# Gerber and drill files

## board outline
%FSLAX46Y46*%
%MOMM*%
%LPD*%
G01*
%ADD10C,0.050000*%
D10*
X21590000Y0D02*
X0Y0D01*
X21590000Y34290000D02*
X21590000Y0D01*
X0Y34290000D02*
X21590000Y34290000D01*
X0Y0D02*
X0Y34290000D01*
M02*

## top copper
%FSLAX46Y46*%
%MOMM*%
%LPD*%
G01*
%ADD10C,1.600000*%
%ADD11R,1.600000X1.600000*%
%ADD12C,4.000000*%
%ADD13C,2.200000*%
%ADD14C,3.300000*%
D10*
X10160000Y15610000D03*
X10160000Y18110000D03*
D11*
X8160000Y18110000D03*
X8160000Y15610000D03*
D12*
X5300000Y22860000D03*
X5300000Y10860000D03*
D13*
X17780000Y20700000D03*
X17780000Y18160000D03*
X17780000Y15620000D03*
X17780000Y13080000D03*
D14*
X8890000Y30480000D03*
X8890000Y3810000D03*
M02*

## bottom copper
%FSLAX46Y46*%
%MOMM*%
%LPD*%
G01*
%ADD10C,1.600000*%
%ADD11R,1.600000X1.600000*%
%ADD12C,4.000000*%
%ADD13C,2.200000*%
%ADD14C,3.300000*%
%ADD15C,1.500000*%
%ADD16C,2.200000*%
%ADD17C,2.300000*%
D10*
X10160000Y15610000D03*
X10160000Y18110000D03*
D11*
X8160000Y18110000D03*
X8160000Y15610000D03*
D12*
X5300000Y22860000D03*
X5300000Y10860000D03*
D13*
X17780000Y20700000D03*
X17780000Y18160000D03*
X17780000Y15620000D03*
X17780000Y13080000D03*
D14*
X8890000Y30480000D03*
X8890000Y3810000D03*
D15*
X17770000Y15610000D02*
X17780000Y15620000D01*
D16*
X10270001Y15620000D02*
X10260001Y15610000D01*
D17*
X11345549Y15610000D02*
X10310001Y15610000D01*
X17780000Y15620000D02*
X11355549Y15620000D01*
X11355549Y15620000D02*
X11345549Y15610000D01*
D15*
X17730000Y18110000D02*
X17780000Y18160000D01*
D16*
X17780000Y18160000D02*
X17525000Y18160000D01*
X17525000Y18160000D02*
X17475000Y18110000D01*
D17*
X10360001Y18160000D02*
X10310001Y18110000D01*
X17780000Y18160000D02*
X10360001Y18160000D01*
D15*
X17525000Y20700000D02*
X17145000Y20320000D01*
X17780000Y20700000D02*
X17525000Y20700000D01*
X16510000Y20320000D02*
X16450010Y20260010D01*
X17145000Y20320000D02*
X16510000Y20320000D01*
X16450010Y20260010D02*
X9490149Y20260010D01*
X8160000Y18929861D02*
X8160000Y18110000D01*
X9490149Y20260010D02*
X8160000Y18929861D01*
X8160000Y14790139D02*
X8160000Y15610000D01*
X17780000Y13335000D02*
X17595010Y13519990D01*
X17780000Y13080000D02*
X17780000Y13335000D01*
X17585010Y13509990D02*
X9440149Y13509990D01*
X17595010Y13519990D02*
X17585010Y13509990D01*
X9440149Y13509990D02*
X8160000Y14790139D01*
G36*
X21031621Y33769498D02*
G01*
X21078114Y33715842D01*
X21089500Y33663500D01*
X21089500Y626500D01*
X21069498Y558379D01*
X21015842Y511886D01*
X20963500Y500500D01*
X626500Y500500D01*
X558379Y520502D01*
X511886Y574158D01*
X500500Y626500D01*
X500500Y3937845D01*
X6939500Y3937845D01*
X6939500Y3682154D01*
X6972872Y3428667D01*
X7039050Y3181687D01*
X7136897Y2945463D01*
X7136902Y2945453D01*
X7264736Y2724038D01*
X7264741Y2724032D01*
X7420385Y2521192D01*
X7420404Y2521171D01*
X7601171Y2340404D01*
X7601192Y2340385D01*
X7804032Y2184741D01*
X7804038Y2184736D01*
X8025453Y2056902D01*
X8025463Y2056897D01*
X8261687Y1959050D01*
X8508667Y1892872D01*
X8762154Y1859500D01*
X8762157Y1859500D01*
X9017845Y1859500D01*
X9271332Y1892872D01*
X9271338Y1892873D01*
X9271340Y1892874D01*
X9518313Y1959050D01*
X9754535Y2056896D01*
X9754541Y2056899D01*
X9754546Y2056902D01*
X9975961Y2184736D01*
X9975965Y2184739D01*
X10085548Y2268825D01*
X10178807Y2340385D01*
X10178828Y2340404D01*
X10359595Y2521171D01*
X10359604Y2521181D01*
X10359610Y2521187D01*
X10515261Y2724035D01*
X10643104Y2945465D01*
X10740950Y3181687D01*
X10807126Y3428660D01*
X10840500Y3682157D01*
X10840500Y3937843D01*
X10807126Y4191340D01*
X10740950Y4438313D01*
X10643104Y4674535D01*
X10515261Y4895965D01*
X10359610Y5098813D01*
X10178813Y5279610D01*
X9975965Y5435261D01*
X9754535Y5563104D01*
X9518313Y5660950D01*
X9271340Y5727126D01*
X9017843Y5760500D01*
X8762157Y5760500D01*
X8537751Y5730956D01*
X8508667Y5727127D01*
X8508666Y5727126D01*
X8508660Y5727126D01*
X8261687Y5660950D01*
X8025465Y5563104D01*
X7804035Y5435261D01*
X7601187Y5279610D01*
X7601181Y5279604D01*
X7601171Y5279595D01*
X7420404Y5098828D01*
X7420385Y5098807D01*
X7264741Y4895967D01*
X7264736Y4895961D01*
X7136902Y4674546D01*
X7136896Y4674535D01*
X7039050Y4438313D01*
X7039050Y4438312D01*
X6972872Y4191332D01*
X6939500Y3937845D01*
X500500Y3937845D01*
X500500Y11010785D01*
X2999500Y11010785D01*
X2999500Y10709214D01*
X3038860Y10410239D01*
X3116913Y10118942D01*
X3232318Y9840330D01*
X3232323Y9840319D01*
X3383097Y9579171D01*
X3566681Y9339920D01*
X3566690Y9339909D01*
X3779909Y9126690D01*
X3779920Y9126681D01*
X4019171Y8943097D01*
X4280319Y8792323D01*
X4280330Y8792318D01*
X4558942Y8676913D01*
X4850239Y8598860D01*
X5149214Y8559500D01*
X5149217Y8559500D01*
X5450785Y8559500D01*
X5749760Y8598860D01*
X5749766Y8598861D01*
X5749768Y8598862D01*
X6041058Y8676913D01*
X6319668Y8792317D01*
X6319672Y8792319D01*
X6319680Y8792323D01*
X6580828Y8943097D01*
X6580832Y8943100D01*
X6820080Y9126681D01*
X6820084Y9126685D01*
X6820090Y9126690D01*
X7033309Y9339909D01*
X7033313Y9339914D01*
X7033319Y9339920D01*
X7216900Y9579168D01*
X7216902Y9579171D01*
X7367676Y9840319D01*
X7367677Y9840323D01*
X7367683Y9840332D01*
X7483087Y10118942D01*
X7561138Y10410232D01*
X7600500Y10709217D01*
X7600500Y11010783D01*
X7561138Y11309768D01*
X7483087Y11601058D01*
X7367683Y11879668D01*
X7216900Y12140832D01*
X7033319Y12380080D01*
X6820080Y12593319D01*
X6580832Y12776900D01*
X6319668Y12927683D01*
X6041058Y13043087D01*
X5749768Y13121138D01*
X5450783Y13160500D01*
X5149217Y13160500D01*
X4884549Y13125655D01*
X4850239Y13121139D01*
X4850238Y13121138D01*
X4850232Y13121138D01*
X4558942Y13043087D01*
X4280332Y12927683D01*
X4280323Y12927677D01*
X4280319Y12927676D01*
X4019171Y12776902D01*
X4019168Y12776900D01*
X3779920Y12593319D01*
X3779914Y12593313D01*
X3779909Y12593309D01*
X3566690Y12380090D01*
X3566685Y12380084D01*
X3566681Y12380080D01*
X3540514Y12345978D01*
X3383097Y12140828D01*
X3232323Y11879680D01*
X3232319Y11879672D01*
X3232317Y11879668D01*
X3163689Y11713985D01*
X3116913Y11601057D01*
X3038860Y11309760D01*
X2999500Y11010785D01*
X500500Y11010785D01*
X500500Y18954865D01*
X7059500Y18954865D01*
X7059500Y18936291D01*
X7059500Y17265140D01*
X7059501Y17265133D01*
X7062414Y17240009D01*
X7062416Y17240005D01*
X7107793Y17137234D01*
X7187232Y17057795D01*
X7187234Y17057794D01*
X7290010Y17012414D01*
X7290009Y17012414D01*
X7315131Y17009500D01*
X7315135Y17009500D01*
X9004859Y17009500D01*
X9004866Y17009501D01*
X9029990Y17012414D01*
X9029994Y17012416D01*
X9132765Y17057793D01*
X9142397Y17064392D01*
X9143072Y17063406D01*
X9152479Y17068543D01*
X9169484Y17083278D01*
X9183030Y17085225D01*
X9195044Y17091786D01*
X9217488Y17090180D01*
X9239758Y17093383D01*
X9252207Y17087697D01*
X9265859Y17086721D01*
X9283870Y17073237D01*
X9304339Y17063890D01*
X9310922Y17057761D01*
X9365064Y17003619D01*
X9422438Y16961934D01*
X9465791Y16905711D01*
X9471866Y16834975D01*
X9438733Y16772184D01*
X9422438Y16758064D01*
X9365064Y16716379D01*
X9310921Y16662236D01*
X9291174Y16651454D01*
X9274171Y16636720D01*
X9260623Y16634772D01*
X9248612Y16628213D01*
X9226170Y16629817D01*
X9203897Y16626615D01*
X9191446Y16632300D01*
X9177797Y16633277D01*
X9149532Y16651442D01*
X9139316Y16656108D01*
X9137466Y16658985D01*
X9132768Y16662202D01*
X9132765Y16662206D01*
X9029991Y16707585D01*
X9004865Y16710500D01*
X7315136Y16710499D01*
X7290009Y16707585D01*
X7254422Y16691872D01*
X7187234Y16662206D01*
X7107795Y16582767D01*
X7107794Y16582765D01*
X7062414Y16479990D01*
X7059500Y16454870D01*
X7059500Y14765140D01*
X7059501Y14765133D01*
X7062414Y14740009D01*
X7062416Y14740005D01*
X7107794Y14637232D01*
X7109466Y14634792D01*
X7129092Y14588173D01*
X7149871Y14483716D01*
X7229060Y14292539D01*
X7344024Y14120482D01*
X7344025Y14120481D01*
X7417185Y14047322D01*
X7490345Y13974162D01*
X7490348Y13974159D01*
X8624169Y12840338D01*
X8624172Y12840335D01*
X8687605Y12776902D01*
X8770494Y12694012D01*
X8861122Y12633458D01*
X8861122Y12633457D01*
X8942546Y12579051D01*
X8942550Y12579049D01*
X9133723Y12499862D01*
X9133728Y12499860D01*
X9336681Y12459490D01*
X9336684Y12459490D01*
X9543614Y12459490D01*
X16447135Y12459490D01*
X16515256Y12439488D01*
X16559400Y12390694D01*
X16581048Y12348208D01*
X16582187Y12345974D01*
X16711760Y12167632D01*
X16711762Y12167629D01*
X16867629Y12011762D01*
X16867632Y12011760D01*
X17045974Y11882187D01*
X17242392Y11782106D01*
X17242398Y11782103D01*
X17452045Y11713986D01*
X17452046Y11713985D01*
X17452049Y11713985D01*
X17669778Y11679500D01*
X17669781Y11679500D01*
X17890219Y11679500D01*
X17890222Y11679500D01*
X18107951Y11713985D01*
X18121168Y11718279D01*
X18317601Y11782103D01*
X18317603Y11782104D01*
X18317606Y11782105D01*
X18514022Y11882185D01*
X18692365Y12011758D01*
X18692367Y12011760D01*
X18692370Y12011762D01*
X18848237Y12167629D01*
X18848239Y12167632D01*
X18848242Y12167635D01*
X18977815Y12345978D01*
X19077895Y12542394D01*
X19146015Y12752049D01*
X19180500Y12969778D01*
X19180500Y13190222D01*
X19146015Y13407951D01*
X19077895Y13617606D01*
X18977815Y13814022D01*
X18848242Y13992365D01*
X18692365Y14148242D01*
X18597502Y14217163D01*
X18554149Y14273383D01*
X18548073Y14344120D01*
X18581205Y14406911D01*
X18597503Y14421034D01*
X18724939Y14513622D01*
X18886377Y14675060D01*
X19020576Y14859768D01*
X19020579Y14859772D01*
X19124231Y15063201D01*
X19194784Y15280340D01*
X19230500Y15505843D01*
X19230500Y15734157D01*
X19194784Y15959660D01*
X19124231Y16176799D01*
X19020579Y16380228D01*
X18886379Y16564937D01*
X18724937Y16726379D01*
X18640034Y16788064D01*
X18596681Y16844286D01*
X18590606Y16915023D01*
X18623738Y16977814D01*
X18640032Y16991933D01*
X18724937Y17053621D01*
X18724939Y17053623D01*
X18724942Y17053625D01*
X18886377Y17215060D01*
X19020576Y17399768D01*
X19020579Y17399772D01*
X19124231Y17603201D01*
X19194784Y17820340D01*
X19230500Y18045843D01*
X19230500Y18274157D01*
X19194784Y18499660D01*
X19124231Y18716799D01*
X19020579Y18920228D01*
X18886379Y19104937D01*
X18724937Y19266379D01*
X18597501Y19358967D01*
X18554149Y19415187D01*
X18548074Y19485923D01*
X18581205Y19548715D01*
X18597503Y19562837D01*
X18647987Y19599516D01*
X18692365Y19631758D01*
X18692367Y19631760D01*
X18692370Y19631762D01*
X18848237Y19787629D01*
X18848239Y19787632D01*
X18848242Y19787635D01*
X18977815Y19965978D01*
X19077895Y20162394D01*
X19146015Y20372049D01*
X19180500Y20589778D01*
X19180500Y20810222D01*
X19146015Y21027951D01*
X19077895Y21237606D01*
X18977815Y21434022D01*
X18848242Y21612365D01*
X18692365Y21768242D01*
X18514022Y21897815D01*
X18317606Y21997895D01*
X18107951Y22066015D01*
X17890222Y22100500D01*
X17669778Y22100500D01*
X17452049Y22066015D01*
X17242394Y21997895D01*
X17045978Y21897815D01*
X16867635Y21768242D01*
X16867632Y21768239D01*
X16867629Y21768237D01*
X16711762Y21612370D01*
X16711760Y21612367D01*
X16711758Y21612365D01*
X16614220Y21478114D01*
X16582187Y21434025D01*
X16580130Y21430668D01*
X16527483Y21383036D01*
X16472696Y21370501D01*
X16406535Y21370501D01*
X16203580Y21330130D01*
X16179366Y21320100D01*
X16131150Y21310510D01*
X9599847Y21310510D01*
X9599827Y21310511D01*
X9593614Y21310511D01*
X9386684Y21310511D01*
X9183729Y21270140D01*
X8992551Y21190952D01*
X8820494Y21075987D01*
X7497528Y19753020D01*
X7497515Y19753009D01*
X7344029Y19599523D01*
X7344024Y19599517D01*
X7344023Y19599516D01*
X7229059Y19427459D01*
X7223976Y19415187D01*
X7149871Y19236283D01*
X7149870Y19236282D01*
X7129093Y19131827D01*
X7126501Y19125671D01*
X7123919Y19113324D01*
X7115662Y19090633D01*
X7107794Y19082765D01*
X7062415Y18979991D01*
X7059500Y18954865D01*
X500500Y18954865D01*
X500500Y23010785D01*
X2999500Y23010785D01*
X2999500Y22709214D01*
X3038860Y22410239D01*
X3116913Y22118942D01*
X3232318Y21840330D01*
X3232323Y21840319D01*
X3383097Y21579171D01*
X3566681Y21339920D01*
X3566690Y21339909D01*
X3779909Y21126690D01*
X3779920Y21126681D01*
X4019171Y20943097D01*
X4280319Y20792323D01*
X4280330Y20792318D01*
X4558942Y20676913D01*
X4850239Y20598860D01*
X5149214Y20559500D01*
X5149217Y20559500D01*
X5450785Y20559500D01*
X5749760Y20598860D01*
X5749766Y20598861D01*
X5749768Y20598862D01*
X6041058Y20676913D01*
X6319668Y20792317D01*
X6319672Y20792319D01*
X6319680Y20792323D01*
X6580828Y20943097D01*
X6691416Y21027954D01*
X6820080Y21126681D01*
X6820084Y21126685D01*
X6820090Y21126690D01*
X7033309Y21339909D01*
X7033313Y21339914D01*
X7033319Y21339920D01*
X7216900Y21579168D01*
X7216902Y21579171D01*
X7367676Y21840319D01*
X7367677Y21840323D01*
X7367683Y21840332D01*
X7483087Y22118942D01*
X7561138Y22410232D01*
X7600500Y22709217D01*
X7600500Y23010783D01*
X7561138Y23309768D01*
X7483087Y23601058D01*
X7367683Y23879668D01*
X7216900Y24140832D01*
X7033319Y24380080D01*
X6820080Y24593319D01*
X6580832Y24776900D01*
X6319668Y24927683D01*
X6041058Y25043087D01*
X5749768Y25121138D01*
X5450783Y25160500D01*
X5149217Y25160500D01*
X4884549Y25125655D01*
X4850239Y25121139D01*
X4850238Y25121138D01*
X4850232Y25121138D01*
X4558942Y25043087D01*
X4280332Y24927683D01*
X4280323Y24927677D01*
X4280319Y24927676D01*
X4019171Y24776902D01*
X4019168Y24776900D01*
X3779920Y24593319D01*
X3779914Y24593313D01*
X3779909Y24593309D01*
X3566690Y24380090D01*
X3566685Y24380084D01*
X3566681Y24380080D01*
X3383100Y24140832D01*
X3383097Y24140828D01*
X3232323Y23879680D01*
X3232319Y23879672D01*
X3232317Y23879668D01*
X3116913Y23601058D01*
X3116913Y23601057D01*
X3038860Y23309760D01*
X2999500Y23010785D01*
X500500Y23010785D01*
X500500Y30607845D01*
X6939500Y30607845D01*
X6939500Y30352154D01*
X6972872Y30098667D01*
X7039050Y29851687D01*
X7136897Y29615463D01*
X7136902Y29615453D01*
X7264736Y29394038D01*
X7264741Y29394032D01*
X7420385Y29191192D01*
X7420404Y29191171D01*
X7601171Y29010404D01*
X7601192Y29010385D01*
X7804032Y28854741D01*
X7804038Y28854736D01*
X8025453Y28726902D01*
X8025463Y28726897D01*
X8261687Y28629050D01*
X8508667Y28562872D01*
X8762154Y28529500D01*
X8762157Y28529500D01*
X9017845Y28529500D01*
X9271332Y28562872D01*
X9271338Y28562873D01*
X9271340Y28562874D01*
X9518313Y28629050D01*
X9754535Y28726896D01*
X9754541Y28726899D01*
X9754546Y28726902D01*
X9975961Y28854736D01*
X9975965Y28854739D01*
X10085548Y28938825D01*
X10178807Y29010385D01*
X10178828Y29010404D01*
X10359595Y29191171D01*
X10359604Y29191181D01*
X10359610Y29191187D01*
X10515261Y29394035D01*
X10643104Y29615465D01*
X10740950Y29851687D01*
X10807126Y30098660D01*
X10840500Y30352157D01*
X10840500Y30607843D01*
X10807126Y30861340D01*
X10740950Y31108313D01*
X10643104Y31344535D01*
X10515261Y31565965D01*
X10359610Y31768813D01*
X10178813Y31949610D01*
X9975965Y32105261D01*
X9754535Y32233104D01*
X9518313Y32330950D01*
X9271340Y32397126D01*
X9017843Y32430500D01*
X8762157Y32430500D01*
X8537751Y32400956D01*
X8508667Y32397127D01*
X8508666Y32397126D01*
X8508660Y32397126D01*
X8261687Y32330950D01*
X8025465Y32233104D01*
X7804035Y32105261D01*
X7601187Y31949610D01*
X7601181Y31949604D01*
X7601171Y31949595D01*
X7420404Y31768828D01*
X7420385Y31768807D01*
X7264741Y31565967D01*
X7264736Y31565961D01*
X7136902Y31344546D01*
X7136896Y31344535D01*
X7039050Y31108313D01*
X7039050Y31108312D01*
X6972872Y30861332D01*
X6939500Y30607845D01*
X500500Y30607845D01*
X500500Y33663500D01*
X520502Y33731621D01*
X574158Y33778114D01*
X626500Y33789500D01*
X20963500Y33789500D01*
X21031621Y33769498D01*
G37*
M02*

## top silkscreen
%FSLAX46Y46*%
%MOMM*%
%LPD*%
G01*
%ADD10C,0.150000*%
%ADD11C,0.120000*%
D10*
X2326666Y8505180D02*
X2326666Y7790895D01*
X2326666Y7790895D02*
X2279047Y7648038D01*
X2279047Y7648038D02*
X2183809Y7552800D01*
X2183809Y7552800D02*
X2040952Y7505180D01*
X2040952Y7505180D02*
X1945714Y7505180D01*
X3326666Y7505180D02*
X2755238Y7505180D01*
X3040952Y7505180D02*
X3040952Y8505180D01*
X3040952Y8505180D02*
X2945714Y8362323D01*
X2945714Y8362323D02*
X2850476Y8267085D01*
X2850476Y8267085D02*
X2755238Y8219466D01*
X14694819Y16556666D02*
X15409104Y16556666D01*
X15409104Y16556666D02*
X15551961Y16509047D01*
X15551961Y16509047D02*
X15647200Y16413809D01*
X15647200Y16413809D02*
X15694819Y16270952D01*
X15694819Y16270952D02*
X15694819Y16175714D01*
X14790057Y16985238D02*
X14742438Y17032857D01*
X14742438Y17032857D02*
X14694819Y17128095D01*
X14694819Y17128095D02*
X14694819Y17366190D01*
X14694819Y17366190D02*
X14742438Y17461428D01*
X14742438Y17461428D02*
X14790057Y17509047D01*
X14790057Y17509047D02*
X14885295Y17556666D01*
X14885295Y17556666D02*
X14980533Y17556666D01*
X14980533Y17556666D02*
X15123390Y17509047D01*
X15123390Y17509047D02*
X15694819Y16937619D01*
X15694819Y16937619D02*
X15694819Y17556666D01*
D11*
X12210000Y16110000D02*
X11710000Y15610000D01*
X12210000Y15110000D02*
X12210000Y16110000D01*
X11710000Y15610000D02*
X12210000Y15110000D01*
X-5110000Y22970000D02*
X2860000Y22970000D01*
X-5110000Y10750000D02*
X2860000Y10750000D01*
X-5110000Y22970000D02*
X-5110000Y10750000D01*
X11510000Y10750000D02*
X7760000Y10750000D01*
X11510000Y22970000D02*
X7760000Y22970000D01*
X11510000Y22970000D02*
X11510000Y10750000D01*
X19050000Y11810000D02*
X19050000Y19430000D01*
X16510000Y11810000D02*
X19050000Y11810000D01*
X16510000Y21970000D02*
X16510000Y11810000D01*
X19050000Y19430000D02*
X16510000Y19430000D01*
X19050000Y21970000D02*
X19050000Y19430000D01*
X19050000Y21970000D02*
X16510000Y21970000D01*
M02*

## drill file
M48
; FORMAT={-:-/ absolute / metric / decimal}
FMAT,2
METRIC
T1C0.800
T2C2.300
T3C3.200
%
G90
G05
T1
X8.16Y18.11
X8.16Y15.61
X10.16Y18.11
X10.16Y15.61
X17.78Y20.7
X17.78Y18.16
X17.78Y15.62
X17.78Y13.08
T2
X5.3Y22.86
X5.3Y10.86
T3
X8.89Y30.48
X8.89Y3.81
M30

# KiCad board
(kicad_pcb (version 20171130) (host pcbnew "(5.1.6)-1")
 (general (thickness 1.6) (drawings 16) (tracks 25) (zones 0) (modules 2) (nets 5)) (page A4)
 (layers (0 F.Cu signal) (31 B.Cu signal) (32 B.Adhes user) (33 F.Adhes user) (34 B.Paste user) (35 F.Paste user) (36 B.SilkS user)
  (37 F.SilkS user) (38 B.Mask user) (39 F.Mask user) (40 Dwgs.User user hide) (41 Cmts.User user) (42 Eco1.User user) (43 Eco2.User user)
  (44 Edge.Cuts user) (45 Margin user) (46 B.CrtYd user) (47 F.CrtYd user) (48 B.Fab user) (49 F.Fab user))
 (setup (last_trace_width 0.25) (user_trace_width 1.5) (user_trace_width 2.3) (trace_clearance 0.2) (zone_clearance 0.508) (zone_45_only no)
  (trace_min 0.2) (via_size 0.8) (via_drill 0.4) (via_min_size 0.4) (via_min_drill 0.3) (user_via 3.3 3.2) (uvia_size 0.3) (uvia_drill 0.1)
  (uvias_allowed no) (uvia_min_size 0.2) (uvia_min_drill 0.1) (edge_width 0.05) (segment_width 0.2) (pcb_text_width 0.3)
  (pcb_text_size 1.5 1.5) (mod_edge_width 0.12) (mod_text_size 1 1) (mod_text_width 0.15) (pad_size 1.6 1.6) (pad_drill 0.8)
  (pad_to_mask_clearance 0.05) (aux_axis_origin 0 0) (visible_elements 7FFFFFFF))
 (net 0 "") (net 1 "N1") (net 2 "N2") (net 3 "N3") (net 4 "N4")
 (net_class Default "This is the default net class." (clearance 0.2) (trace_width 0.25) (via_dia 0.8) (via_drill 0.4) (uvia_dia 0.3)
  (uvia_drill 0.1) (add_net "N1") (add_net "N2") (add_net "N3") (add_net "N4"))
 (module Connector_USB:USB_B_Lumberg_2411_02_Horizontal (layer F.Cu) (at 10.16 -15.61 180)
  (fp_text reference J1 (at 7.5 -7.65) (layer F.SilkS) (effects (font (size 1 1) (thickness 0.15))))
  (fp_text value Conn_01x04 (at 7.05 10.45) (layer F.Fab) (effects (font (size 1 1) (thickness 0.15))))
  (fp_line (start -2.05 0.5) (end -1.55 0) (layer F.SilkS) (width 0.12))
  (fp_line (start -2.05 -0.5) (end -2.05 0.5) (layer F.SilkS) (width 0.12))
  (fp_line (start -1.55 0) (end -2.05 -0.5) (layer F.SilkS) (width 0.12))
  (fp_line (start 15.27 7.36) (end 7.3 7.36) (layer F.SilkS) (width 0.12))
  (fp_line (start 15.27 -4.86) (end 7.3 -4.86) (layer F.SilkS) (width 0.12))
  (fp_line (start 15.27 7.36) (end 15.27 -4.86) (layer F.SilkS) (width 0.12))
  (fp_line (start -1.35 -4.86) (end 2.4 -4.86) (layer F.SilkS) (width 0.12))
  (fp_line (start -1.35 7.36) (end 2.4 7.36) (layer F.SilkS) (width 0.12))
  (fp_line (start -1.35 7.36) (end -1.35 -4.86) (layer F.SilkS) (width 0.12))
  (pad 1 thru_hole circle (at 0 0 270) (size 1.6 1.6) (drill 0.8) (layers *.Cu *.Mask) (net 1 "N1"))
  (pad 2 thru_hole circle (at 0 2.5 270) (size 1.6 1.6) (drill 0.8) (layers *.Cu *.Mask) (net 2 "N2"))
  (pad 3 thru_hole rect (at 2 2.5 270) (size 1.6 1.6) (drill 0.8) (layers *.Cu *.Mask) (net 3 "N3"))
  (pad 4 thru_hole rect (at 2 0 270) (size 1.6 1.6) (drill 0.8) (layers *.Cu *.Mask) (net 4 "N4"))
  (pad 5 thru_hole circle (at 4.86 7.25 270) (size 4 4) (drill 2.3) (layers *.Cu *.Mask))
  (pad 5 thru_hole circle (at 4.86 -4.75 270) (size 4 4) (drill 2.3) (layers *.Cu *.Mask)))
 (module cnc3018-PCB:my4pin (layer F.Cu) (at 17.78 -20.7 270)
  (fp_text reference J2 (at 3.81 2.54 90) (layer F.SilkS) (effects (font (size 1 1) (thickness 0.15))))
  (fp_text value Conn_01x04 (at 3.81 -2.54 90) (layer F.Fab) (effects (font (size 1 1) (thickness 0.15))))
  (fp_line (start 8.89 -1.27) (end 1.27 -1.27) (layer F.SilkS) (width 0.12))
  (fp_line (start 8.89 1.27) (end 8.89 -1.27) (layer F.SilkS) (width 0.12))
  (fp_line (start -1.27 1.27) (end 8.89 1.27) (layer F.SilkS) (width 0.12))
  (fp_line (start 1.27 -1.27) (end 1.27 1.27) (layer F.SilkS) (width 0.12))
  (fp_line (start -1.27 -1.27) (end 1.27 -1.27) (layer F.SilkS) (width 0.12))
  (fp_line (start -1.27 -1.27) (end -1.27 1.27) (layer F.SilkS) (width 0.12))
  (pad 1 thru_hole circle (at 0 0 270) (size 2.2 2.2) (drill 0.8) (layers *.Cu *.Mask) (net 3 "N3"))
  (pad 2 thru_hole circle (at 2.54 0 270) (size 2.2 2.2) (drill 0.8) (layers *.Cu *.Mask) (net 2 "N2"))
  (pad 3 thru_hole circle (at 5.08 0 270) (size 2.2 2.2) (drill 0.8) (layers *.Cu *.Mask) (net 1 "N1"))
  (pad 4 thru_hole circle (at 7.62 0 270) (size 2.2 2.2) (drill 0.8) (layers *.Cu *.Mask) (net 4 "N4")))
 (gr_line (start 21.59 0) (end 0 0) (layer Edge.Cuts) (width 0.05))
 (gr_line (start 21.59 -34.29) (end 21.59 0) (layer Edge.Cuts) (width 0.05))
 (gr_line (start 0 -34.29) (end 21.59 -34.29) (layer Edge.Cuts) (width 0.05))
 (gr_line (start 0 0) (end 0 -34.29) (layer Edge.Cuts) (width 0.05))
 (via (at 8.89 -30.48) (size 3.3) (drill 3.2) (layers F.Cu B.Cu) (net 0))
 (via (at 8.89 -3.81) (size 3.3) (drill 3.2) (layers F.Cu B.Cu) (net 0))
 (segment (start 17.77 -15.61) (end 17.78 -15.62) (width 1.5) (layer B.Cu) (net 1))
 (segment (start 10.270001 -15.62) (end 10.260001 -15.61) (width 2.2) (layer B.Cu) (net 1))
 (segment (start 11.345549 -15.61) (end 10.310001 -15.61) (width 2.3) (layer B.Cu) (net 1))
 (segment (start 17.78 -15.62) (end 11.355549 -15.62) (width 2.3) (layer B.Cu) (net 1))
 (segment (start 11.355549 -15.62) (end 11.345549 -15.61) (width 2.3) (layer B.Cu) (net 1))
 (segment (start 17.73 -18.11) (end 17.78 -18.16) (width 1.5) (layer B.Cu) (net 2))
 (segment (start 17.78 -18.16) (end 17.525 -18.16) (width 2.2) (layer B.Cu) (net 2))
 (segment (start 17.525 -18.16) (end 17.475 -18.11) (width 2.2) (layer B.Cu) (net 2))
 (segment (start 10.360001 -18.16) (end 10.310001 -18.11) (width 2.3) (layer B.Cu) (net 2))
 (segment (start 17.78 -18.16) (end 10.360001 -18.16) (width 2.3) (layer B.Cu) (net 2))
 (segment (start 17.525 -20.7) (end 17.145 -20.32) (width 1.5) (layer B.Cu) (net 3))
 (segment (start 17.78 -20.7) (end 17.525 -20.7) (width 1.5) (layer B.Cu) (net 3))
 (segment (start 16.51 -20.32) (end 16.45001 -20.26001) (width 1.5) (layer B.Cu) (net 3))
 (segment (start 17.145 -20.32) (end 16.51 -20.32) (width 1.5) (layer B.Cu) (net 3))
 (segment (start 16.45001 -20.26001) (end 9.490149 -20.26001) (width 1.5) (layer B.Cu) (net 3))
 (segment (start 8.16 -18.929861) (end 8.16 -18.11) (width 1.5) (layer B.Cu) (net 3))
 (segment (start 9.490149 -20.26001) (end 8.16 -18.929861) (width 1.5) (layer B.Cu) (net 3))
 (segment (start 8.16 -14.790139) (end 8.16 -15.61) (width 1.5) (layer B.Cu) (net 4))
 (segment (start 17.78 -13.335) (end 17.59501 -13.51999) (width 1.5) (layer B.Cu) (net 4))
 (segment (start 17.78 -13.08) (end 17.78 -13.335) (width 1.5) (layer B.Cu) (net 4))
 (segment (start 17.58501 -13.50999) (end 9.440149 -13.50999) (width 1.5) (layer B.Cu) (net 4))
 (segment (start 17.59501 -13.51999) (end 17.58501 -13.50999) (width 1.5) (layer B.Cu) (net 4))
 (segment (start 9.440149 -13.50999) (end 8.16 -14.790139) (width 1.5) (layer B.Cu) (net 4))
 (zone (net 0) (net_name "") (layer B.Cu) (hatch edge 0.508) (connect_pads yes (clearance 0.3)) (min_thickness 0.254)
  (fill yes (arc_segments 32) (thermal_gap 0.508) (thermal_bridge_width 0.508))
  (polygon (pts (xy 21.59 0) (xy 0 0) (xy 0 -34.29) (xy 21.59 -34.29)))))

